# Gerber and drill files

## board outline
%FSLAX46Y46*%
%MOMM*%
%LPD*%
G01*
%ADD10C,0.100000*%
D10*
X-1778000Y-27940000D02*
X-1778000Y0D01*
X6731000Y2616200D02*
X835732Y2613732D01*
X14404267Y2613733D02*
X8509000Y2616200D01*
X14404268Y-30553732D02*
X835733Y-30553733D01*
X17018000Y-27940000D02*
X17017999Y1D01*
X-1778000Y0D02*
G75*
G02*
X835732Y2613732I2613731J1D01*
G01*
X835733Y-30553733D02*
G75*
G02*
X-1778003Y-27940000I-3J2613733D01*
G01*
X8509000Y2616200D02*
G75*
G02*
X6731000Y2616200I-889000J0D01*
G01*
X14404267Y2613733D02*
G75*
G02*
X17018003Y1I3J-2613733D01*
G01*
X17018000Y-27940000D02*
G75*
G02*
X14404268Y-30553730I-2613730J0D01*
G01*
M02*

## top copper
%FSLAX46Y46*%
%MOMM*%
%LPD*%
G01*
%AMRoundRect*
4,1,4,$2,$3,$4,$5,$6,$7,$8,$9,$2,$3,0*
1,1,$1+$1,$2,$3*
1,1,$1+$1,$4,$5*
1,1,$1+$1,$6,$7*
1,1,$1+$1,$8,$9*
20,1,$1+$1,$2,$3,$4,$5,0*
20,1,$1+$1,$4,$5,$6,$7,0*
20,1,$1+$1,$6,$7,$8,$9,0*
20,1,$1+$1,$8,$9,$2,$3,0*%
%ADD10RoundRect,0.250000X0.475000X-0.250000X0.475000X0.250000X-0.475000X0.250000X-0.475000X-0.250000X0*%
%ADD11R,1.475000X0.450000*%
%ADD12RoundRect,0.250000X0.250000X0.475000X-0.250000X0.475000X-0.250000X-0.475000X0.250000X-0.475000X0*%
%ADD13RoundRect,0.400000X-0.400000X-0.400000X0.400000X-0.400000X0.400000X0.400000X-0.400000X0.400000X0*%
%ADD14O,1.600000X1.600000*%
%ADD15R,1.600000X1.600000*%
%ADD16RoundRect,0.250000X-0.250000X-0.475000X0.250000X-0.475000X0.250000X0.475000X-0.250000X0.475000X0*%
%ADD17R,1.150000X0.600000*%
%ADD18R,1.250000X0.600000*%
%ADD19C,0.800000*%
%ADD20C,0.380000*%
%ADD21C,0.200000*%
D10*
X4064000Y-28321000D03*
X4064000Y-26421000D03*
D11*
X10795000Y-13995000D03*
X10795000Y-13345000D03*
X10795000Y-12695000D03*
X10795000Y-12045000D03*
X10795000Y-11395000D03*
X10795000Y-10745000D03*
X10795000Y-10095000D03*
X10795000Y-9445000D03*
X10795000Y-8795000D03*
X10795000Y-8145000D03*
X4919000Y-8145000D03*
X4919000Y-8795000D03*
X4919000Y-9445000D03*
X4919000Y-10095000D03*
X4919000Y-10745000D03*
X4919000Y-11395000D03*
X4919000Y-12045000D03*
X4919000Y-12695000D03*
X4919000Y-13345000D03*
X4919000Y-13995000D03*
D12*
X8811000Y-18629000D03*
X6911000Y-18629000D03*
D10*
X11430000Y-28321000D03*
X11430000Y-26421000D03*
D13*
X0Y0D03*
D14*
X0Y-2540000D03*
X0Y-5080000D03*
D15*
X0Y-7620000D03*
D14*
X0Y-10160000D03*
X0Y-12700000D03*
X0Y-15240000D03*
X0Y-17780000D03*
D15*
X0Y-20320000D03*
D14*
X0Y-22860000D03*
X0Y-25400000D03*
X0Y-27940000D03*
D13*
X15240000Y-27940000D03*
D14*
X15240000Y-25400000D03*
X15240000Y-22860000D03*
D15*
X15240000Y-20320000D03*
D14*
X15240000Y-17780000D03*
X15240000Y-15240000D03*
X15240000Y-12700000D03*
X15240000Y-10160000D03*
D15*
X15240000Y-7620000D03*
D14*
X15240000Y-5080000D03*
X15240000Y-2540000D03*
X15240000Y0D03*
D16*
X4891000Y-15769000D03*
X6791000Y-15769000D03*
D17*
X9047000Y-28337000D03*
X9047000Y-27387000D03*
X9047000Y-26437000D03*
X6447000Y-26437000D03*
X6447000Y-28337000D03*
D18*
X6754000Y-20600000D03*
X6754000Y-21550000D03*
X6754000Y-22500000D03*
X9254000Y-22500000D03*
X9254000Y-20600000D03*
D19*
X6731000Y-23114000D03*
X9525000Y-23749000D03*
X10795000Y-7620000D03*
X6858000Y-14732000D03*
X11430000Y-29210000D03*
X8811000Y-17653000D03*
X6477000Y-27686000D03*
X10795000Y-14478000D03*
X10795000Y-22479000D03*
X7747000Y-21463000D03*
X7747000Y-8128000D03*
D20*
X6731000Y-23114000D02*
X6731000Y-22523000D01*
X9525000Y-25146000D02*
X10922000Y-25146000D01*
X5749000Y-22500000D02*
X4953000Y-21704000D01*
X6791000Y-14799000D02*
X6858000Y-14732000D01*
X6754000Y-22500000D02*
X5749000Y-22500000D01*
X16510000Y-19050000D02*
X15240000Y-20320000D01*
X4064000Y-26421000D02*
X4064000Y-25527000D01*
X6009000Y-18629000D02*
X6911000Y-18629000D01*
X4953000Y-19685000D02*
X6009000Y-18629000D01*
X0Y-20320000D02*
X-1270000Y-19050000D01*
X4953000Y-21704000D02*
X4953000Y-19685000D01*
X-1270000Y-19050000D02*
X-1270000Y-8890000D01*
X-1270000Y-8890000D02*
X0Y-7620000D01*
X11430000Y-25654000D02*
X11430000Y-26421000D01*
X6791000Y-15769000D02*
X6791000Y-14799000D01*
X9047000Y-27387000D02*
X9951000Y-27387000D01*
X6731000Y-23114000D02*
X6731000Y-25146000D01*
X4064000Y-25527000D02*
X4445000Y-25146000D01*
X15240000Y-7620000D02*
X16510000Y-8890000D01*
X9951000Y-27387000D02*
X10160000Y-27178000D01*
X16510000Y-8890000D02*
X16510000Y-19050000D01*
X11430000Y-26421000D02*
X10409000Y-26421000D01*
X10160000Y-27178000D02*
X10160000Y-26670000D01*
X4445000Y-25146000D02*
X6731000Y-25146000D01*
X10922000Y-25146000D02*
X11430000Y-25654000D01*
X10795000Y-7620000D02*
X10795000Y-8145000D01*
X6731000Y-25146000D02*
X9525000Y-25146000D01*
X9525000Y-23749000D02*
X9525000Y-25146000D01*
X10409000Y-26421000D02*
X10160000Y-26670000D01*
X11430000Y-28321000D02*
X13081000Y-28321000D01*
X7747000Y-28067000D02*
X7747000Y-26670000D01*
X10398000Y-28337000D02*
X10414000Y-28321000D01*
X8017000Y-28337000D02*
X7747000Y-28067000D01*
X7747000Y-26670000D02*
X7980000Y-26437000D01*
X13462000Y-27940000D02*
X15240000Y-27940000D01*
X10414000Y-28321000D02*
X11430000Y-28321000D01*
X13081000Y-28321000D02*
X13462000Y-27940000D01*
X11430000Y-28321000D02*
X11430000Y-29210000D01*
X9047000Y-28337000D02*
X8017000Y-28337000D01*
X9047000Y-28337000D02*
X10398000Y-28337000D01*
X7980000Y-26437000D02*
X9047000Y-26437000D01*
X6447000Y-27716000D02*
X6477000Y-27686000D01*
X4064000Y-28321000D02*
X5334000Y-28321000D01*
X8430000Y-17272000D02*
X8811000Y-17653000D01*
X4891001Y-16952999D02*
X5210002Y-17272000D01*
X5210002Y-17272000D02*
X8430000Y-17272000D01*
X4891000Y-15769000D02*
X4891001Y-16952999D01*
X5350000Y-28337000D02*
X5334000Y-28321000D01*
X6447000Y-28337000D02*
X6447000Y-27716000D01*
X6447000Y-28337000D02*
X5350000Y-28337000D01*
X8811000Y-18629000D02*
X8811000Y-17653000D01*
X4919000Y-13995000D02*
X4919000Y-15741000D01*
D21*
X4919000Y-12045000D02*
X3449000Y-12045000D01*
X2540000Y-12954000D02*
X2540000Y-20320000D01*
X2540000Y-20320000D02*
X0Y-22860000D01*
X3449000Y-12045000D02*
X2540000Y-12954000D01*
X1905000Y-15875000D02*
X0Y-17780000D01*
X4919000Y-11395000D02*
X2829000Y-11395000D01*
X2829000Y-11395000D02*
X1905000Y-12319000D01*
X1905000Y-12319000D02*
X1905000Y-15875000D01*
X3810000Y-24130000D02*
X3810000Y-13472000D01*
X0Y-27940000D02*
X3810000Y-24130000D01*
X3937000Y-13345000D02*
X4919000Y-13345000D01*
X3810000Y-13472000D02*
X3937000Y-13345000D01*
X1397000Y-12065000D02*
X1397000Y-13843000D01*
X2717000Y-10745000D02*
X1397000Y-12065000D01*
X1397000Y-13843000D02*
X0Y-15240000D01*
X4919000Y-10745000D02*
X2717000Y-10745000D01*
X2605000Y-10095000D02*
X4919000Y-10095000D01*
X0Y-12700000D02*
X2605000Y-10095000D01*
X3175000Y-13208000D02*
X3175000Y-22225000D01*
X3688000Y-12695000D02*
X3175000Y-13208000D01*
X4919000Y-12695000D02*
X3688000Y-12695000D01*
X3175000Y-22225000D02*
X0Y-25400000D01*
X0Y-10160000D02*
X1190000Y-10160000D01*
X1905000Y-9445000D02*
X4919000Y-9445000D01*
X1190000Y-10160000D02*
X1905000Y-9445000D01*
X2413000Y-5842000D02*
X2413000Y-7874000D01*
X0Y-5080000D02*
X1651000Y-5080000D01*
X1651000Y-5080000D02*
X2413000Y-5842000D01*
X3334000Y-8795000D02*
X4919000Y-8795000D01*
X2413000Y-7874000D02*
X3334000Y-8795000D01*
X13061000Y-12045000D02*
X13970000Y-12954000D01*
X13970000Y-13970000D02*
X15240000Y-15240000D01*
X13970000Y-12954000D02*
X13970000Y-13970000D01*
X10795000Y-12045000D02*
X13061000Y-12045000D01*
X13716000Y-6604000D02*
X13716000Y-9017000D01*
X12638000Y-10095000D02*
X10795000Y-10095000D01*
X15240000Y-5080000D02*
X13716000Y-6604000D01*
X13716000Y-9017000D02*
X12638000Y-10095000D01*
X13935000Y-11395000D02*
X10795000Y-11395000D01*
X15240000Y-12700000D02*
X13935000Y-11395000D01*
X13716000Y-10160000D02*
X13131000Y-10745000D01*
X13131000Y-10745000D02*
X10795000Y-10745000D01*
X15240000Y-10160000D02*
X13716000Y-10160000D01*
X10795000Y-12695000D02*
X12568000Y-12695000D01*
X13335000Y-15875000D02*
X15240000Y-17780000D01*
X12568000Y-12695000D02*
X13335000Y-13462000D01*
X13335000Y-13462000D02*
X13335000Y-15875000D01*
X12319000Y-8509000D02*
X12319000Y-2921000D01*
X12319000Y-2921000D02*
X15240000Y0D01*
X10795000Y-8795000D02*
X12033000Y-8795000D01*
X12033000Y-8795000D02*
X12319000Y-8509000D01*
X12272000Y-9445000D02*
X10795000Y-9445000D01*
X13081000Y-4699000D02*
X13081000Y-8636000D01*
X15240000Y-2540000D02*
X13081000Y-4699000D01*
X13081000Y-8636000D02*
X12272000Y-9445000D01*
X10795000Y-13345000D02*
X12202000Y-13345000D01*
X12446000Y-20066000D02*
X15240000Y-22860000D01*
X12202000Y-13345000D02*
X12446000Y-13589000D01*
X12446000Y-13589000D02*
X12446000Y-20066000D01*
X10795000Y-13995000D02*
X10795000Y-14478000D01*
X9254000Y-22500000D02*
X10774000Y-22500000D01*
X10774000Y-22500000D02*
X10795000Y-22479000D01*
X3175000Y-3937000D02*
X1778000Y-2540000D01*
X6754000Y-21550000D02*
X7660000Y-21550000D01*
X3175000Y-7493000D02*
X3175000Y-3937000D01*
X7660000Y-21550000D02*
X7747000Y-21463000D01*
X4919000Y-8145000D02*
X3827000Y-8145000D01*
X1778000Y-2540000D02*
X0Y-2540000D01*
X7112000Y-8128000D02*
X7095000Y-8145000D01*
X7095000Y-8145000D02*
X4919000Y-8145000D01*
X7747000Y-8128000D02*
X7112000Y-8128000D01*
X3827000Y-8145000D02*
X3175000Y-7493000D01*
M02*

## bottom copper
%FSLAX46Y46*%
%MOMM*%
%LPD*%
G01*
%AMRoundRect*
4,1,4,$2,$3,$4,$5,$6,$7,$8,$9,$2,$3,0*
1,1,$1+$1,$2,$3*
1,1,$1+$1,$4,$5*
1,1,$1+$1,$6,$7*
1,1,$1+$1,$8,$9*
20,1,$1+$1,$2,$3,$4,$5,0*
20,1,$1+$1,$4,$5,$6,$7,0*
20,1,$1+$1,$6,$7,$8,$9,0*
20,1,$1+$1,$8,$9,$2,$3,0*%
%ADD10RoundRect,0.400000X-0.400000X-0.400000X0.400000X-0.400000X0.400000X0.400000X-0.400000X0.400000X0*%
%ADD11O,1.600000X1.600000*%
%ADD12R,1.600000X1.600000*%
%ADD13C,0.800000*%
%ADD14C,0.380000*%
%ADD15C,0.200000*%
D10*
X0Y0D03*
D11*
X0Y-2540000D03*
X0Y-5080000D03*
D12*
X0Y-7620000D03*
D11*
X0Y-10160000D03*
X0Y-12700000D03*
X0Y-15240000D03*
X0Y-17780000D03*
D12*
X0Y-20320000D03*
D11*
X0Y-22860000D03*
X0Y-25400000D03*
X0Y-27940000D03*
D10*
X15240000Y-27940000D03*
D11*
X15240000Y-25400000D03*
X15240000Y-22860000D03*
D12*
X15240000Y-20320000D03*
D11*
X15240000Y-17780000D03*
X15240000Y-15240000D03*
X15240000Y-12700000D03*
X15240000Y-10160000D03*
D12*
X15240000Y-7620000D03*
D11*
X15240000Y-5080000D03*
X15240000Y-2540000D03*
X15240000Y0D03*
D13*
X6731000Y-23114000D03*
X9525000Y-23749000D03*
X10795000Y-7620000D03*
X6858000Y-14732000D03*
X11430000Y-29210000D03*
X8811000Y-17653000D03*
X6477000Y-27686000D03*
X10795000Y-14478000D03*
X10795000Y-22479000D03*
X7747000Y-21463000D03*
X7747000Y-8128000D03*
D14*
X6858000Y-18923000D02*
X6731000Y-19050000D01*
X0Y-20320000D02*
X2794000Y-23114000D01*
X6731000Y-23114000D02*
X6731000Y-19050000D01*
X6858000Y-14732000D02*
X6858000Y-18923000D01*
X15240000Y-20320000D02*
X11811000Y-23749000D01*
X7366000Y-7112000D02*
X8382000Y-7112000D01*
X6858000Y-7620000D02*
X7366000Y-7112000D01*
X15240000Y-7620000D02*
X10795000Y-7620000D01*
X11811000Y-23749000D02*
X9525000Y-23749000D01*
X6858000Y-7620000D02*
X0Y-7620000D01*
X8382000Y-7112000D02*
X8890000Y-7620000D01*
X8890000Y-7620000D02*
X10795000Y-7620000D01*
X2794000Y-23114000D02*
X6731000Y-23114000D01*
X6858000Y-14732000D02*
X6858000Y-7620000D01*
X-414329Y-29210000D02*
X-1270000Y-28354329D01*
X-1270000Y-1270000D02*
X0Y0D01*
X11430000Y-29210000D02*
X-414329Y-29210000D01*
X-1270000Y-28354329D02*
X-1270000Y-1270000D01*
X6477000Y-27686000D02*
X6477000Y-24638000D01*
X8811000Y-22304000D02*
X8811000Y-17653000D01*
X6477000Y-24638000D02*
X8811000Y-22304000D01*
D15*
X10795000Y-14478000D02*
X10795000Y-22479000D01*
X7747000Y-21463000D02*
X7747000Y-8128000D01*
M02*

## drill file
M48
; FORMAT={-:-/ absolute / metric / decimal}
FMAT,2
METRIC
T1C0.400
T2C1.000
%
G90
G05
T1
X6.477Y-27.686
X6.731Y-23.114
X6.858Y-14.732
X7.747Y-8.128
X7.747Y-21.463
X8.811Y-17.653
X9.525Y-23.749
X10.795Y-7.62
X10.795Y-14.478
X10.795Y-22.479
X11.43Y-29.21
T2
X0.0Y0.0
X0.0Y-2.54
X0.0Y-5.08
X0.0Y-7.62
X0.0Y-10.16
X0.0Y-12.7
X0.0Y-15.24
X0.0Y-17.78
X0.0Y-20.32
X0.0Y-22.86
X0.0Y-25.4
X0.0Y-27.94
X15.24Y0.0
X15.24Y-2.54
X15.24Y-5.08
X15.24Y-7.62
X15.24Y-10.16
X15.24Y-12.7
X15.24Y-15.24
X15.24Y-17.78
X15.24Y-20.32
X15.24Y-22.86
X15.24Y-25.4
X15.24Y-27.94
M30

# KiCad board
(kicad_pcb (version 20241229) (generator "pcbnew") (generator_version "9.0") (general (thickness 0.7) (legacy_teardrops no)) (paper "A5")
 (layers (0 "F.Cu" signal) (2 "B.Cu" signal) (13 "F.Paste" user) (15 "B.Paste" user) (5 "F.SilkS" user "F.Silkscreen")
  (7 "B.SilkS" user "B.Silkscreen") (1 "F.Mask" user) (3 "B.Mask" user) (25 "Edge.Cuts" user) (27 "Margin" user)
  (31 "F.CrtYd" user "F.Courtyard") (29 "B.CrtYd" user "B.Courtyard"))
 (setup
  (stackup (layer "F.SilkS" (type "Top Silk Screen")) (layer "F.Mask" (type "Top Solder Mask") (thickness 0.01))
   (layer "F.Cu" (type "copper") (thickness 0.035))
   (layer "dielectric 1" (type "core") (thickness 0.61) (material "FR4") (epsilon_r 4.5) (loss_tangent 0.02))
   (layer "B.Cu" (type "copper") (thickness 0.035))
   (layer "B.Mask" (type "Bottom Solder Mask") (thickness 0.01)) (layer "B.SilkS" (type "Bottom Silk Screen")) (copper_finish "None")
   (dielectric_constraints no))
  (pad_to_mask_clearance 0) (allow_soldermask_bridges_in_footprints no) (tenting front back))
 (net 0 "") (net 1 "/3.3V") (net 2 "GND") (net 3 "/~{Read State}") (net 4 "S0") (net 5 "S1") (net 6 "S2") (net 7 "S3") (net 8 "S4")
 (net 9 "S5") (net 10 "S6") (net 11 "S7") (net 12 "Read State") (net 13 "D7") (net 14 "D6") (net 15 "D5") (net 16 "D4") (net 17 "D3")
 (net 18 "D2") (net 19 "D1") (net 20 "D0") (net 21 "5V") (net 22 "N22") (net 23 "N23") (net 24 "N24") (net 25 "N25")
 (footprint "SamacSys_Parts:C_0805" (layer "F.Cu") (at 4.064 27.387)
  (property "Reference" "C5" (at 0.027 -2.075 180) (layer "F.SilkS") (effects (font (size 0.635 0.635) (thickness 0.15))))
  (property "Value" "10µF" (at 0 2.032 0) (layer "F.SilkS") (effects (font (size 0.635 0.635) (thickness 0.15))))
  (pad "1" smd roundrect (at 0 0.934 90) (size 1 1.45) (layers "F.Cu" "F.Mask" "F.Paste") (roundrect_rratio 0.25) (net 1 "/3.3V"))
  (pad "2" smd roundrect (at 0 -0.966 90) (size 1 1.45) (layers "F.Cu" "F.Mask" "F.Paste") (roundrect_rratio 0.25) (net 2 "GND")))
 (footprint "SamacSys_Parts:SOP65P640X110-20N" (layer "F.Cu") (at 7.857 11.07 180)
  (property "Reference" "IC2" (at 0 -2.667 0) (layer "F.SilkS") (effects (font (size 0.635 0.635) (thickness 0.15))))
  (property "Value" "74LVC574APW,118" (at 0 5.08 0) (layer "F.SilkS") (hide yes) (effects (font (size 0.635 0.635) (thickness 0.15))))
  (pad "1" smd rect (at -2.938 -2.925 270) (size 0.45 1.475) (layers "F.Cu" "F.Mask" "F.Paste") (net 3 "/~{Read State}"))
  (pad "2" smd rect (at -2.938 -2.275 270) (size 0.45 1.475) (layers "F.Cu" "F.Mask" "F.Paste") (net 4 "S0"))
  (pad "3" smd rect (at -2.938 -1.625 270) (size 0.45 1.475) (layers "F.Cu" "F.Mask" "F.Paste") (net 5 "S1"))
  (pad "4" smd rect (at -2.938 -0.975 270) (size 0.45 1.475) (layers "F.Cu" "F.Mask" "F.Paste") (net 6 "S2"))
  (pad "5" smd rect (at -2.938 -0.325 270) (size 0.45 1.475) (layers "F.Cu" "F.Mask" "F.Paste") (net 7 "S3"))
  (pad "6" smd rect (at -2.938 0.325 270) (size 0.45 1.475) (layers "F.Cu" "F.Mask" "F.Paste") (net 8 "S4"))
  (pad "7" smd rect (at -2.938 0.975 270) (size 0.45 1.475) (layers "F.Cu" "F.Mask" "F.Paste") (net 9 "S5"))
  (pad "8" smd rect (at -2.938 1.625 270) (size 0.45 1.475) (layers "F.Cu" "F.Mask" "F.Paste") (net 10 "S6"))
  (pad "9" smd rect (at -2.938 2.275 270) (size 0.45 1.475) (layers "F.Cu" "F.Mask" "F.Paste") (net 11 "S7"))
  (pad "10" smd rect (at -2.938 2.925 270) (size 0.45 1.475) (layers "F.Cu" "F.Mask" "F.Paste") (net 2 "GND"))
  (pad "11" smd rect (at 2.938 2.925 270) (size 0.45 1.475) (layers "F.Cu" "F.Mask" "F.Paste") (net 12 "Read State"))
  (pad "12" smd rect (at 2.938 2.275 270) (size 0.45 1.475) (layers "F.Cu" "F.Mask" "F.Paste") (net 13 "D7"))
  (pad "13" smd rect (at 2.938 1.625 270) (size 0.45 1.475) (layers "F.Cu" "F.Mask" "F.Paste") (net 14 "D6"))
  (pad "14" smd rect (at 2.938 0.975 270) (size 0.45 1.475) (layers "F.Cu" "F.Mask" "F.Paste") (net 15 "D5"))
  (pad "15" smd rect (at 2.938 0.325 270) (size 0.45 1.475) (layers "F.Cu" "F.Mask" "F.Paste") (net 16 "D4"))
  (pad "16" smd rect (at 2.938 -0.325 270) (size 0.45 1.475) (layers "F.Cu" "F.Mask" "F.Paste") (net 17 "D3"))
  (pad "17" smd rect (at 2.938 -0.975 270) (size 0.45 1.475) (layers "F.Cu" "F.Mask" "F.Paste") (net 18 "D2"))
  (pad "18" smd rect (at 2.938 -1.625 270) (size 0.45 1.475) (layers "F.Cu" "F.Mask" "F.Paste") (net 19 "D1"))
  (pad "19" smd rect (at 2.938 -2.275 270) (size 0.45 1.475) (layers "F.Cu" "F.Mask" "F.Paste") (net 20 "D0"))
  (pad "20" smd rect (at 2.938 -2.925 270) (size 0.45 1.475) (layers "F.Cu" "F.Mask" "F.Paste") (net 1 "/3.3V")))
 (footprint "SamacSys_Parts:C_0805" (layer "F.Cu") (at 7.877 18.629 90)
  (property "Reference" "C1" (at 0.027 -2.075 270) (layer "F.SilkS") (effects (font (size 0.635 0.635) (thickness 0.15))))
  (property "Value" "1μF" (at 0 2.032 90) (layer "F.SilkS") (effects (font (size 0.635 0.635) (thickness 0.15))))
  (pad "1" smd roundrect (at 0 0.934 180) (size 1 1.45) (layers "F.Cu" "F.Mask" "F.Paste") (roundrect_rratio 0.25) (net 1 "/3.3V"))
  (pad "2" smd roundrect (at 0 -0.966 180) (size 1 1.45) (layers "F.Cu" "F.Mask" "F.Paste") (roundrect_rratio 0.25) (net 2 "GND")))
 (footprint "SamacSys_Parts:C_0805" (layer "F.Cu") (at 11.43 27.387)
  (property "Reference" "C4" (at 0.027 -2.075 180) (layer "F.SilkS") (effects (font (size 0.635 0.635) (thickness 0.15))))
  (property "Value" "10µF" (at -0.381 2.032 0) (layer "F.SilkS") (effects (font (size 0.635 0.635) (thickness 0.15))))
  (pad "1" smd roundrect (at 0 0.934 90) (size 1 1.45) (layers "F.Cu" "F.Mask" "F.Paste") (roundrect_rratio 0.25) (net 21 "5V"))
  (pad "2" smd roundrect (at 0 -0.966 90) (size 1 1.45) (layers "F.Cu" "F.Mask" "F.Paste") (roundrect_rratio 0.25) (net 2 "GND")))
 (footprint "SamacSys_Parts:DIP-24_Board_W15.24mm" (layer "F.Cu") (at 0 0)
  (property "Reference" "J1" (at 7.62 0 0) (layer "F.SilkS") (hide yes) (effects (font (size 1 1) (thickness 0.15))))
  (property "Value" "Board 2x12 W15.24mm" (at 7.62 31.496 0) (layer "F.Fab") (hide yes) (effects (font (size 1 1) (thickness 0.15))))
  (fp_line (start -1.778 27.94) (end -1.778 0) (stroke (width 0.1) (type solid)) (layer "Edge.Cuts"))
  (fp_line (start 6.731 -2.6162) (end 0.835732 -2.613732) (stroke (width 0.1) (type solid)) (layer "Edge.Cuts"))
  (fp_line (start 14.404267 -2.613733) (end 8.509 -2.6162) (stroke (width 0.1) (type solid)) (layer "Edge.Cuts"))
  (fp_line (start 14.404268 30.553732) (end 0.835733 30.553733) (stroke (width 0.1) (type solid)) (layer "Edge.Cuts"))
  (fp_line (start 17.018 27.94) (end 17.017999 -0.000001) (stroke (width 0.1) (type solid)) (layer "Edge.Cuts"))
  (fp_arc (start -1.778 0) (mid -1.012456 -1.848188) (end 0.835732 -2.613732) (stroke (width 0.1) (type solid)) (layer "Edge.Cuts"))
  (fp_arc (start 0.835733 30.553733) (mid -1.012456 29.788189) (end -1.778 27.94) (stroke (width 0.1) (type solid)) (layer "Edge.Cuts"))
  (fp_arc (start 8.509 -2.6162) (mid 7.62 -1.7272) (end 6.731 -2.6162) (stroke (width 0.1) (type default)) (layer "Edge.Cuts"))
  (fp_arc (start 14.404267 -2.613733) (mid 16.252455 -1.848189) (end 17.017999 -0.000001) (stroke (width 0.1) (type solid))
   (layer "Edge.Cuts"))
  (fp_arc (start 17.018 27.94) (mid 16.252455 29.788187) (end 14.404268 30.553732) (stroke (width 0.1) (type solid)) (layer "Edge.Cuts"))
  (pad "1" thru_hole roundrect (at 0 0) (size 1.6 1.6) (drill 1) (layers "*.Cu" "*.Mask") (remove_unused_layers no) (roundrect_rratio 0.25)
   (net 21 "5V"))
  (pad "2" thru_hole oval (at 0 2.54) (size 1.6 1.6) (drill 1) (layers "*.Cu" "*.Mask") (remove_unused_layers no) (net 12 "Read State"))
  (pad "3" thru_hole oval (at 0 5.08) (size 1.6 1.6) (drill 1) (layers "*.Cu" "*.Mask") (remove_unused_layers no) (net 13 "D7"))
  (pad "4" thru_hole rect (at 0 7.62) (size 1.6 1.6) (drill 1) (layers "*.Cu" "*.Mask") (remove_unused_layers no) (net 2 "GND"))
  (pad "5" thru_hole oval (at 0 10.16) (size 1.6 1.6) (drill 1) (layers "*.Cu" "*.Mask") (remove_unused_layers no) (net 14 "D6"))
  (pad "6" thru_hole oval (at 0 12.7) (size 1.6 1.6) (drill 1) (layers "*.Cu" "*.Mask") (remove_unused_layers no) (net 15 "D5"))
  (pad "7" thru_hole oval (at 0 15.24) (size 1.6 1.6) (drill 1) (layers "*.Cu" "*.Mask") (remove_unused_layers no) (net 16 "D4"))
  (pad "8" thru_hole oval (at 0 17.78) (size 1.6 1.6) (drill 1) (layers "*.Cu" "*.Mask") (remove_unused_layers no) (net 17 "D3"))
  (pad "9" thru_hole rect (at 0 20.32) (size 1.6 1.6) (drill 1) (layers "*.Cu" "*.Mask") (remove_unused_layers no) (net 2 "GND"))
  (pad "10" thru_hole oval (at 0 22.86) (size 1.6 1.6) (drill 1) (layers "*.Cu" "*.Mask") (remove_unused_layers no) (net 18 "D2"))
  (pad "11" thru_hole oval (at 0 25.4) (size 1.6 1.6) (drill 1) (layers "*.Cu" "*.Mask") (remove_unused_layers no) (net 19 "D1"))
  (pad "12" thru_hole oval (at 0 27.94) (size 1.6 1.6) (drill 1) (layers "*.Cu" "*.Mask") (remove_unused_layers no) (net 20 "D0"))
  (pad "13" thru_hole roundrect (at 15.24 27.94) (size 1.6 1.6) (drill 1) (layers "*.Cu" "*.Mask") (remove_unused_layers no)
   (roundrect_rratio 0.25) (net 21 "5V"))
  (pad "14" thru_hole oval (at 15.24 25.4) (size 1.6 1.6) (drill 1) (layers "*.Cu" "*.Mask") (remove_unused_layers no) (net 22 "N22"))
  (pad "15" thru_hole oval (at 15.24 22.86) (size 1.6 1.6) (drill 1) (layers "*.Cu" "*.Mask") (remove_unused_layers no) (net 4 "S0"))
  (pad "16" thru_hole rect (at 15.24 20.32) (size 1.6 1.6) (drill 1) (layers "*.Cu" "*.Mask") (remove_unused_layers no) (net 2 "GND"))
  (pad "17" thru_hole oval (at 15.24 17.78 180) (size 1.6 1.6) (drill 1) (layers "*.Cu" "*.Mask") (remove_unused_layers no) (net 5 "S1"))
  (pad "18" thru_hole oval (at 15.24 15.24 180) (size 1.6 1.6) (drill 1) (layers "*.Cu" "*.Mask") (remove_unused_layers no) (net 6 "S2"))
  (pad "19" thru_hole oval (at 15.24 12.7 180) (size 1.6 1.6) (drill 1) (layers "*.Cu" "*.Mask") (remove_unused_layers no) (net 7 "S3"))
  (pad "20" thru_hole oval (at 15.24 10.16 180) (size 1.6 1.6) (drill 1) (layers "*.Cu" "*.Mask") (remove_unused_layers no) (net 8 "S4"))
  (pad "21" thru_hole rect (at 15.24 7.62) (size 1.6 1.6) (drill 1) (layers "*.Cu" "*.Mask") (remove_unused_layers no) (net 2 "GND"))
  (pad "22" thru_hole oval (at 15.24 5.08) (size 1.6 1.6) (drill 1) (layers "*.Cu" "*.Mask") (remove_unused_layers no) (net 9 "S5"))
  (pad "23" thru_hole oval (at 15.24 2.54) (size 1.6 1.6) (drill 1) (layers "*.Cu" "*.Mask") (remove_unused_layers no) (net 10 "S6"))
  (pad "24" thru_hole oval (at 15.24 0) (size 1.6 1.6) (drill 1) (layers "*.Cu" "*.Mask") (remove_unused_layers no) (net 11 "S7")))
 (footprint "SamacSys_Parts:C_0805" (layer "F.Cu") (at 5.825 15.769 -90)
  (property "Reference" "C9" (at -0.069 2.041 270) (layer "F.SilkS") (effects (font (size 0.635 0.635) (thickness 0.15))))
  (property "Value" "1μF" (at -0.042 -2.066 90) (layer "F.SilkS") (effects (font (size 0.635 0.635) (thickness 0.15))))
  (pad "1" smd roundrect (at 0 0.934) (size 1 1.45) (layers "F.Cu" "F.Mask" "F.Paste") (roundrect_rratio 0.25) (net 1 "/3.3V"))
  (pad "2" smd roundrect (at 0 -0.966) (size 1 1.45) (layers "F.Cu" "F.Mask" "F.Paste") (roundrect_rratio 0.25) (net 2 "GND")))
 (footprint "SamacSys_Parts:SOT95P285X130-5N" (layer "F.Cu") (at 7.747 27.387 180)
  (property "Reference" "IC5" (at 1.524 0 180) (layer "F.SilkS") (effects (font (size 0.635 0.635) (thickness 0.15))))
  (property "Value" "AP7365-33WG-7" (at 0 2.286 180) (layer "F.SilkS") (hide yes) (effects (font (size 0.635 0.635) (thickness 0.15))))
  (pad "1" smd rect (at -1.3 -0.95 270) (size 0.6 1.15) (layers "F.Cu" "F.Mask" "F.Paste") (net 21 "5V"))
  (pad "2" smd rect (at -1.3 0 270) (size 0.6 1.15) (layers "F.Cu" "F.Mask" "F.Paste") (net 2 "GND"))
  (pad "3" smd rect (at -1.3 0.95 270) (size 0.6 1.15) (layers "F.Cu" "F.Mask" "F.Paste") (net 21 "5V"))
  (pad "4" smd rect (at 1.3 0.95 270) (size 0.6 1.15) (layers "F.Cu" "F.Mask" "F.Paste") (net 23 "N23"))
  (pad "5" smd rect (at 1.3 -0.95 270) (size 0.6 1.15) (layers "F.Cu" "F.Mask" "F.Paste") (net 1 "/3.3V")))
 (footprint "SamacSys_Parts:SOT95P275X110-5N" (layer "F.Cu") (at 8.004 21.55)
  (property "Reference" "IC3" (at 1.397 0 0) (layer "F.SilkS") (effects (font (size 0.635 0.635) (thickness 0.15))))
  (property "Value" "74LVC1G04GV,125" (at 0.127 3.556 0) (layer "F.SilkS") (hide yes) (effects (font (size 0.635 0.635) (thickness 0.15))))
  (pad "1" smd rect (at -1.25 -0.95 90) (size 0.6 1.25) (layers "F.Cu" "F.Mask" "F.Paste") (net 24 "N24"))
  (pad "2" smd rect (at -1.25 0 90) (size 0.6 1.25) (layers "F.Cu" "F.Mask" "F.Paste") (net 12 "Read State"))
  (pad "3" smd rect (at -1.25 0.95 90) (size 0.6 1.25) (layers "F.Cu" "F.Mask" "F.Paste") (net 2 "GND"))
  (pad "4" smd rect (at 1.25 0.95 90) (size 0.6 1.25) (layers "F.Cu" "F.Mask" "F.Paste") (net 3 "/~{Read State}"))
  (pad "5" smd rect (at 1.25 -0.95 90) (size 0.6 1.25) (layers "F.Cu" "F.Mask" "F.Paste") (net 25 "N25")))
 (segment (start 6.731 23.114) (end 6.731 22.523) (width 0.38) (layer "F.Cu") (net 2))
 (segment (start 9.525 25.146) (end 10.922 25.146) (width 0.38) (layer "F.Cu") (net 2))
 (segment (start 5.749 22.5) (end 4.953 21.704) (width 0.38) (layer "F.Cu") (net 2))
 (segment (start 6.791 14.799) (end 6.858 14.732) (width 0.38) (layer "F.Cu") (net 2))
 (segment (start 6.754 22.5) (end 5.749 22.5) (width 0.38) (layer "F.Cu") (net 2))
 (segment (start 16.51 19.05) (end 15.24 20.32) (width 0.38) (layer "F.Cu") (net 2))
 (segment (start 4.064 26.421) (end 4.064 25.527) (width 0.38) (layer "F.Cu") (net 2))
 (segment (start 6.009 18.629) (end 6.911 18.629) (width 0.38) (layer "F.Cu") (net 2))
 (segment (start 4.953 19.685) (end 6.009 18.629) (width 0.38) (layer "F.Cu") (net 2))
 (segment (start 0 20.32) (end -1.27 19.05) (width 0.38) (layer "F.Cu") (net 2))
 (segment (start 4.953 21.704) (end 4.953 19.685) (width 0.38) (layer "F.Cu") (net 2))
 (segment (start -1.27 19.05) (end -1.27 8.89) (width 0.38) (layer "F.Cu") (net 2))
 (segment (start -1.27 8.89) (end 0 7.62) (width 0.38) (layer "F.Cu") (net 2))
 (segment (start 11.43 25.654) (end 11.43 26.421) (width 0.38) (layer "F.Cu") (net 2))
 (segment (start 6.791 15.769) (end 6.791 14.799) (width 0.38) (layer "F.Cu") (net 2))
 (segment (start 9.047 27.387) (end 9.951 27.387) (width 0.38) (layer "F.Cu") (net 2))
 (segment (start 6.731 23.114) (end 6.731 25.146) (width 0.38) (layer "F.Cu") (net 2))
 (segment (start 4.064 25.527) (end 4.445 25.146) (width 0.38) (layer "F.Cu") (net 2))
 (segment (start 15.24 7.62) (end 16.51 8.89) (width 0.38) (layer "F.Cu") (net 2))
 (segment (start 9.951 27.387) (end 10.16 27.178) (width 0.38) (layer "F.Cu") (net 2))
 (segment (start 16.51 8.89) (end 16.51 19.05) (width 0.38) (layer "F.Cu") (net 2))
 (segment (start 11.43 26.421) (end 10.409 26.421) (width 0.38) (layer "F.Cu") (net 2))
 (segment (start 10.16 27.178) (end 10.16 26.67) (width 0.38) (layer "F.Cu") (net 2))
 (segment (start 4.445 25.146) (end 6.731 25.146) (width 0.38) (layer "F.Cu") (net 2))
 (segment (start 10.922 25.146) (end 11.43 25.654) (width 0.38) (layer "F.Cu") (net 2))
 (segment (start 10.795 7.62) (end 10.795 8.145) (width 0.38) (layer "F.Cu") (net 2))
 (segment (start 6.731 25.146) (end 9.525 25.146) (width 0.38) (layer "F.Cu") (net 2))
 (segment (start 9.525 23.749) (end 9.525 25.146) (width 0.38) (layer "F.Cu") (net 2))
 (segment (start 10.409 26.421) (end 10.16 26.67) (width 0.38) (layer "F.Cu") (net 2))
 (via (at 6.731 23.114) (size 0.8) (drill 0.4) (layers "F.Cu" "B.Cu") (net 2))
 (via (at 9.525 23.749) (size 0.8) (drill 0.4) (layers "F.Cu" "B.Cu") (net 2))
 (via (at 10.795 7.62) (size 0.8) (drill 0.4) (layers "F.Cu" "B.Cu") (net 2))
 (via (at 6.858 14.732) (size 0.8) (drill 0.4) (layers "F.Cu" "B.Cu") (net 2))
 (segment (start 6.858 18.923) (end 6.731 19.05) (width 0.38) (layer "B.Cu") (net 2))
 (segment (start 0 20.32) (end 2.794 23.114) (width 0.38) (layer "B.Cu") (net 2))
 (segment (start 6.731 23.114) (end 6.731 19.05) (width 0.38) (layer "B.Cu") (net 2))
 (segment (start 6.858 14.732) (end 6.858 18.923) (width 0.38) (layer "B.Cu") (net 2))
 (segment (start 15.24 20.32) (end 11.811 23.749) (width 0.38) (layer "B.Cu") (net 2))
 (segment (start 7.366 7.112) (end 8.382 7.112) (width 0.38) (layer "B.Cu") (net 2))
 (segment (start 6.858 7.62) (end 7.366 7.112) (width 0.38) (layer "B.Cu") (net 2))
 (segment (start 15.24 7.62) (end 10.795 7.62) (width 0.38) (layer "B.Cu") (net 2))
 (segment (start 11.811 23.749) (end 9.525 23.749) (width 0.38) (layer "B.Cu") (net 2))
 (segment (start 6.858 7.62) (end 0 7.62) (width 0.38) (layer "B.Cu") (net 2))
 (segment (start 8.382 7.112) (end 8.89 7.62) (width 0.38) (layer "B.Cu") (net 2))
 (segment (start 8.89 7.62) (end 10.795 7.62) (width 0.38) (layer "B.Cu") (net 2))
 (segment (start 2.794 23.114) (end 6.731 23.114) (width 0.38) (layer "B.Cu") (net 2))
 (segment (start 6.858 14.732) (end 6.858 7.62) (width 0.38) (layer "B.Cu") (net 2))
 (segment (start 11.43 28.321) (end 13.081 28.321) (width 0.38) (layer "F.Cu") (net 21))
 (segment (start 7.747 28.067) (end 7.747 26.67) (width 0.38) (layer "F.Cu") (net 21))
 (segment (start 10.398 28.337) (end 10.414 28.321) (width 0.38) (layer "F.Cu") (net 21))
 (segment (start 8.017 28.337) (end 7.747 28.067) (width 0.38) (layer "F.Cu") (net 21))
 (segment (start 7.747 26.67) (end 7.98 26.437) (width 0.38) (layer "F.Cu") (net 21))
 (segment (start 13.462 27.94) (end 15.24 27.94) (width 0.38) (layer "F.Cu") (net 21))
 (segment (start 10.414 28.321) (end 11.43 28.321) (width 0.38) (layer "F.Cu") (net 21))
 (segment (start 13.081 28.321) (end 13.462 27.94) (width 0.38) (layer "F.Cu") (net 21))
 (segment (start 11.43 28.321) (end 11.43 29.21) (width 0.38) (layer "F.Cu") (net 21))
 (segment (start 9.047 28.337) (end 8.017 28.337) (width 0.38) (layer "F.Cu") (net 21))
 (segment (start 9.047 28.337) (end 10.398 28.337) (width 0.38) (layer "F.Cu") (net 21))
 (segment (start 7.98 26.437) (end 9.047 26.437) (width 0.38) (layer "F.Cu") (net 21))
 (via (at 11.43 29.21) (size 0.8) (drill 0.4) (layers "F.Cu" "B.Cu") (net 21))
 (segment (start -0.414329 29.21) (end -1.27 28.354329) (width 0.38) (layer "B.Cu") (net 21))
 (segment (start -1.27 1.27) (end 0 0) (width 0.38) (layer "B.Cu") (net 21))
 (segment (start 11.43 29.21) (end -0.414329 29.21) (width 0.38) (layer "B.Cu") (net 21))
 (segment (start -1.27 28.354329) (end -1.27 1.27) (width 0.38) (layer "B.Cu") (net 21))
 (segment (start 6.447 27.716) (end 6.477 27.686) (width 0.38) (layer "F.Cu") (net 1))
 (segment (start 4.064 28.321) (end 5.334 28.321) (width 0.38) (layer "F.Cu") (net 1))
 (segment (start 8.43 17.272) (end 8.811 17.653) (width 0.38) (layer "F.Cu") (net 1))
 (segment (start 4.891001 16.952999) (end 5.210002 17.272) (width 0.38) (layer "F.Cu") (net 1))
 (segment (start 5.210002 17.272) (end 8.43 17.272) (width 0.38) (layer "F.Cu") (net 1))
 (segment (start 4.891 15.769) (end 4.891001 16.952999) (width 0.38) (layer "F.Cu") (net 1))
 (segment (start 5.35 28.337) (end 5.334 28.321) (width 0.38) (layer "F.Cu") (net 1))
 (segment (start 6.447 28.337) (end 6.447 27.716) (width 0.38) (layer "F.Cu") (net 1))
 (segment (start 6.447 28.337) (end 5.35 28.337) (width 0.38) (layer "F.Cu") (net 1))
 (segment (start 8.811 18.629) (end 8.811 17.653) (width 0.38) (layer "F.Cu") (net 1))
 (segment (start 4.919 13.995) (end 4.919 15.741) (width 0.38) (layer "F.Cu") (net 1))
 (via (at 8.811 17.653) (size 0.8) (drill 0.4) (layers "F.Cu" "B.Cu") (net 1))
 (via (at 6.477 27.686) (size 0.8) (drill 0.4) (layers "F.Cu" "B.Cu") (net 1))
 (segment (start 6.477 27.686) (end 6.477 24.638) (width 0.38) (layer "B.Cu") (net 1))
 (segment (start 8.811 22.304) (end 8.811 17.653) (width 0.38) (layer "B.Cu") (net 1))
 (segment (start 6.477 24.638) (end 8.811 22.304) (width 0.38) (layer "B.Cu") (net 1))
 (segment (start 4.919 12.045) (end 3.449 12.045) (width 0.2) (layer "F.Cu") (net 18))
 (segment (start 2.54 12.954) (end 2.54 20.32) (width 0.2) (layer "F.Cu") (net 18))
 (segment (start 2.54 20.32) (end 0 22.86) (width 0.2) (layer "F.Cu") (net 18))
 (segment (start 3.449 12.045) (end 2.54 12.954) (width 0.2) (layer "F.Cu") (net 18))
 (segment (start 1.905 15.875) (end 0 17.78) (width 0.2) (layer "F.Cu") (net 17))
 (segment (start 4.919 11.395) (end 2.829 11.395) (width 0.2) (layer "F.Cu") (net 17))
 (segment (start 2.829 11.395) (end 1.905 12.319) (width 0.2) (layer "F.Cu") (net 17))
 (segment (start 1.905 12.319) (end 1.905 15.875) (width 0.2) (layer "F.Cu") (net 17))
 (segment (start 3.81 24.13) (end 3.81 13.472) (width 0.2) (layer "F.Cu") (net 20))
 (segment (start 0 27.94) (end 3.81 24.13) (width 0.2) (layer "F.Cu") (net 20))
 (segment (start 3.937 13.345) (end 4.919 13.345) (width 0.2) (layer "F.Cu") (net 20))
 (segment (start 3.81 13.472) (end 3.937 13.345) (width 0.2) (layer "F.Cu") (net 20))
 (segment (start 1.397 12.065) (end 1.397 13.843) (width 0.2) (layer "F.Cu") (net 16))
 (segment (start 2.717 10.745) (end 1.397 12.065) (width 0.2) (layer "F.Cu") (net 16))
 (segment (start 1.397 13.843) (end 0 15.24) (width 0.2) (layer "F.Cu") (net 16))
 (segment (start 4.919 10.745) (end 2.717 10.745) (width 0.2) (layer "F.Cu") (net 16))
 (segment (start 2.605 10.095) (end 4.919 10.095) (width 0.2) (layer "F.Cu") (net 15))
 (segment (start 0 12.7) (end 2.605 10.095) (width 0.2) (layer "F.Cu") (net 15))
 (segment (start 3.175 13.208) (end 3.175 22.225) (width 0.2) (layer "F.Cu") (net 19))
 (segment (start 3.688 12.695) (end 3.175 13.208) (width 0.2) (layer "F.Cu") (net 19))
 (segment (start 4.919 12.695) (end 3.688 12.695) (width 0.2) (layer "F.Cu") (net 19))
 (segment (start 3.175 22.225) (end 0 25.4) (width 0.2) (layer "F.Cu") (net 19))
 (segment (start 0 10.16) (end 1.19 10.16) (width 0.2) (layer "F.Cu") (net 14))
 (segment (start 1.905 9.445) (end 4.919 9.445) (width 0.2) (layer "F.Cu") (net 14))
 (segment (start 1.19 10.16) (end 1.905 9.445) (width 0.2) (layer "F.Cu") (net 14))
 (segment (start 2.413 5.842) (end 2.413 7.874) (width 0.2) (layer "F.Cu") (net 13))
 (segment (start 0 5.08) (end 1.651 5.08) (width 0.2) (layer "F.Cu") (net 13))
 (segment (start 1.651 5.08) (end 2.413 5.842) (width 0.2) (layer "F.Cu") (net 13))
 (segment (start 3.334 8.795) (end 4.919 8.795) (width 0.2) (layer "F.Cu") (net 13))
 (segment (start 2.413 7.874) (end 3.334 8.795) (width 0.2) (layer "F.Cu") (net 13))
 (segment (start 13.061 12.045) (end 13.97 12.954) (width 0.2) (layer "F.Cu") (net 6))
 (segment (start 13.97 13.97) (end 15.24 15.24) (width 0.2) (layer "F.Cu") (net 6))
 (segment (start 13.97 12.954) (end 13.97 13.97) (width 0.2) (layer "F.Cu") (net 6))
 (segment (start 10.795 12.045) (end 13.061 12.045) (width 0.2) (layer "F.Cu") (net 6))
 (segment (start 13.716 6.604) (end 13.716 9.017) (width 0.2) (layer "F.Cu") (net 9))
 (segment (start 12.638 10.095) (end 10.795 10.095) (width 0.2) (layer "F.Cu") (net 9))
 (segment (start 15.24 5.08) (end 13.716 6.604) (width 0.2) (layer "F.Cu") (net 9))
 (segment (start 13.716 9.017) (end 12.638 10.095) (width 0.2) (layer "F.Cu") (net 9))
 (segment (start 13.935 11.395) (end 10.795 11.395) (width 0.2) (layer "F.Cu") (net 7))
 (segment (start 15.24 12.7) (end 13.935 11.395) (width 0.2) (layer "F.Cu") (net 7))
 (segment (start 13.716 10.16) (end 13.131 10.745) (width 0.2) (layer "F.Cu") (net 8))
 (segment (start 13.131 10.745) (end 10.795 10.745) (width 0.2) (layer "F.Cu") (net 8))
 (segment (start 15.24 10.16) (end 13.716 10.16) (width 0.2) (layer "F.Cu") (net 8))
 (segment (start 10.795 12.695) (end 12.568 12.695) (width 0.2) (layer "F.Cu") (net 5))
 (segment (start 13.335 15.875) (end 15.24 17.78) (width 0.2) (layer "F.Cu") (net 5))
 (segment (start 12.568 12.695) (end 13.335 13.462) (width 0.2) (layer "F.Cu") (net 5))
 (segment (start 13.335 13.462) (end 13.335 15.875) (width 0.2) (layer "F.Cu") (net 5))
 (segment (start 12.319 8.509) (end 12.319 2.921) (width 0.2) (layer "F.Cu") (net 11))
 (segment (start 12.319 2.921) (end 15.24 0) (width 0.2) (layer "F.Cu") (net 11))
 (segment (start 10.795 8.795) (end 12.033 8.795) (width 0.2) (layer "F.Cu") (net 11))
 (segment (start 12.033 8.795) (end 12.319 8.509) (width 0.2) (layer "F.Cu") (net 11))
 (segment (start 12.272 9.445) (end 10.795 9.445) (width 0.2) (layer "F.Cu") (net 10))
 (segment (start 13.081 4.699) (end 13.081 8.636) (width 0.2) (layer "F.Cu") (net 10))
 (segment (start 15.24 2.54) (end 13.081 4.699) (width 0.2) (layer "F.Cu") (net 10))
 (segment (start 13.081 8.636) (end 12.272 9.445) (width 0.2) (layer "F.Cu") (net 10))
 (segment (start 10.795 13.345) (end 12.202 13.345) (width 0.2) (layer "F.Cu") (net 4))
 (segment (start 12.446 20.066) (end 15.24 22.86) (width 0.2) (layer "F.Cu") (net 4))
 (segment (start 12.202 13.345) (end 12.446 13.589) (width 0.2) (layer "F.Cu") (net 4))
 (segment (start 12.446 13.589) (end 12.446 20.066) (width 0.2) (layer "F.Cu") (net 4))
 (segment (start 10.795 13.995) (end 10.795 14.478) (width 0.2) (layer "F.Cu") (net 3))
 (segment (start 9.254 22.5) (end 10.774 22.5) (width 0.2) (layer "F.Cu") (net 3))
 (segment (start 10.774 22.5) (end 10.795 22.479) (width 0.2) (layer "F.Cu") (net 3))
 (via (at 10.795 14.478) (size 0.8) (drill 0.4) (layers "F.Cu" "B.Cu") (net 3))
 (via (at 10.795 22.479) (size 0.8) (drill 0.4) (layers "F.Cu" "B.Cu") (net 3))
 (segment (start 10.795 14.478) (end 10.795 22.479) (width 0.2) (layer "B.Cu") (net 3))
 (segment (start 3.175 3.937) (end 1.778 2.54) (width 0.2) (layer "F.Cu") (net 12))
 (segment (start 6.754 21.55) (end 7.66 21.55) (width 0.2) (layer "F.Cu") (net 12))
 (segment (start 3.175 7.493) (end 3.175 3.937) (width 0.2) (layer "F.Cu") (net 12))
 (segment (start 7.66 21.55) (end 7.747 21.463) (width 0.2) (layer "F.Cu") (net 12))
 (segment (start 4.919 8.145) (end 3.827 8.145) (width 0.2) (layer "F.Cu") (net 12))
 (segment (start 1.778 2.54) (end 0 2.54) (width 0.2) (layer "F.Cu") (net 12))
 (segment (start 7.112 8.128) (end 7.095 8.145) (width 0.2) (layer "F.Cu") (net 12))
 (segment (start 7.095 8.145) (end 4.919 8.145) (width 0.2) (layer "F.Cu") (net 12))
 (segment (start 7.747 8.128) (end 7.112 8.128) (width 0.2) (layer "F.Cu") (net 12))
 (segment (start 3.827 8.145) (end 3.175 7.493) (width 0.2) (layer "F.Cu") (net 12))
 (via (at 7.747 21.463) (size 0.8) (drill 0.4) (layers "F.Cu" "B.Cu") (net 12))
 (via (at 7.747 8.128) (size 0.8) (drill 0.4) (layers "F.Cu" "B.Cu") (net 12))
 (segment (start 7.747 21.463) (end 7.747 8.128) (width 0.2) (layer "B.Cu") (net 12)))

